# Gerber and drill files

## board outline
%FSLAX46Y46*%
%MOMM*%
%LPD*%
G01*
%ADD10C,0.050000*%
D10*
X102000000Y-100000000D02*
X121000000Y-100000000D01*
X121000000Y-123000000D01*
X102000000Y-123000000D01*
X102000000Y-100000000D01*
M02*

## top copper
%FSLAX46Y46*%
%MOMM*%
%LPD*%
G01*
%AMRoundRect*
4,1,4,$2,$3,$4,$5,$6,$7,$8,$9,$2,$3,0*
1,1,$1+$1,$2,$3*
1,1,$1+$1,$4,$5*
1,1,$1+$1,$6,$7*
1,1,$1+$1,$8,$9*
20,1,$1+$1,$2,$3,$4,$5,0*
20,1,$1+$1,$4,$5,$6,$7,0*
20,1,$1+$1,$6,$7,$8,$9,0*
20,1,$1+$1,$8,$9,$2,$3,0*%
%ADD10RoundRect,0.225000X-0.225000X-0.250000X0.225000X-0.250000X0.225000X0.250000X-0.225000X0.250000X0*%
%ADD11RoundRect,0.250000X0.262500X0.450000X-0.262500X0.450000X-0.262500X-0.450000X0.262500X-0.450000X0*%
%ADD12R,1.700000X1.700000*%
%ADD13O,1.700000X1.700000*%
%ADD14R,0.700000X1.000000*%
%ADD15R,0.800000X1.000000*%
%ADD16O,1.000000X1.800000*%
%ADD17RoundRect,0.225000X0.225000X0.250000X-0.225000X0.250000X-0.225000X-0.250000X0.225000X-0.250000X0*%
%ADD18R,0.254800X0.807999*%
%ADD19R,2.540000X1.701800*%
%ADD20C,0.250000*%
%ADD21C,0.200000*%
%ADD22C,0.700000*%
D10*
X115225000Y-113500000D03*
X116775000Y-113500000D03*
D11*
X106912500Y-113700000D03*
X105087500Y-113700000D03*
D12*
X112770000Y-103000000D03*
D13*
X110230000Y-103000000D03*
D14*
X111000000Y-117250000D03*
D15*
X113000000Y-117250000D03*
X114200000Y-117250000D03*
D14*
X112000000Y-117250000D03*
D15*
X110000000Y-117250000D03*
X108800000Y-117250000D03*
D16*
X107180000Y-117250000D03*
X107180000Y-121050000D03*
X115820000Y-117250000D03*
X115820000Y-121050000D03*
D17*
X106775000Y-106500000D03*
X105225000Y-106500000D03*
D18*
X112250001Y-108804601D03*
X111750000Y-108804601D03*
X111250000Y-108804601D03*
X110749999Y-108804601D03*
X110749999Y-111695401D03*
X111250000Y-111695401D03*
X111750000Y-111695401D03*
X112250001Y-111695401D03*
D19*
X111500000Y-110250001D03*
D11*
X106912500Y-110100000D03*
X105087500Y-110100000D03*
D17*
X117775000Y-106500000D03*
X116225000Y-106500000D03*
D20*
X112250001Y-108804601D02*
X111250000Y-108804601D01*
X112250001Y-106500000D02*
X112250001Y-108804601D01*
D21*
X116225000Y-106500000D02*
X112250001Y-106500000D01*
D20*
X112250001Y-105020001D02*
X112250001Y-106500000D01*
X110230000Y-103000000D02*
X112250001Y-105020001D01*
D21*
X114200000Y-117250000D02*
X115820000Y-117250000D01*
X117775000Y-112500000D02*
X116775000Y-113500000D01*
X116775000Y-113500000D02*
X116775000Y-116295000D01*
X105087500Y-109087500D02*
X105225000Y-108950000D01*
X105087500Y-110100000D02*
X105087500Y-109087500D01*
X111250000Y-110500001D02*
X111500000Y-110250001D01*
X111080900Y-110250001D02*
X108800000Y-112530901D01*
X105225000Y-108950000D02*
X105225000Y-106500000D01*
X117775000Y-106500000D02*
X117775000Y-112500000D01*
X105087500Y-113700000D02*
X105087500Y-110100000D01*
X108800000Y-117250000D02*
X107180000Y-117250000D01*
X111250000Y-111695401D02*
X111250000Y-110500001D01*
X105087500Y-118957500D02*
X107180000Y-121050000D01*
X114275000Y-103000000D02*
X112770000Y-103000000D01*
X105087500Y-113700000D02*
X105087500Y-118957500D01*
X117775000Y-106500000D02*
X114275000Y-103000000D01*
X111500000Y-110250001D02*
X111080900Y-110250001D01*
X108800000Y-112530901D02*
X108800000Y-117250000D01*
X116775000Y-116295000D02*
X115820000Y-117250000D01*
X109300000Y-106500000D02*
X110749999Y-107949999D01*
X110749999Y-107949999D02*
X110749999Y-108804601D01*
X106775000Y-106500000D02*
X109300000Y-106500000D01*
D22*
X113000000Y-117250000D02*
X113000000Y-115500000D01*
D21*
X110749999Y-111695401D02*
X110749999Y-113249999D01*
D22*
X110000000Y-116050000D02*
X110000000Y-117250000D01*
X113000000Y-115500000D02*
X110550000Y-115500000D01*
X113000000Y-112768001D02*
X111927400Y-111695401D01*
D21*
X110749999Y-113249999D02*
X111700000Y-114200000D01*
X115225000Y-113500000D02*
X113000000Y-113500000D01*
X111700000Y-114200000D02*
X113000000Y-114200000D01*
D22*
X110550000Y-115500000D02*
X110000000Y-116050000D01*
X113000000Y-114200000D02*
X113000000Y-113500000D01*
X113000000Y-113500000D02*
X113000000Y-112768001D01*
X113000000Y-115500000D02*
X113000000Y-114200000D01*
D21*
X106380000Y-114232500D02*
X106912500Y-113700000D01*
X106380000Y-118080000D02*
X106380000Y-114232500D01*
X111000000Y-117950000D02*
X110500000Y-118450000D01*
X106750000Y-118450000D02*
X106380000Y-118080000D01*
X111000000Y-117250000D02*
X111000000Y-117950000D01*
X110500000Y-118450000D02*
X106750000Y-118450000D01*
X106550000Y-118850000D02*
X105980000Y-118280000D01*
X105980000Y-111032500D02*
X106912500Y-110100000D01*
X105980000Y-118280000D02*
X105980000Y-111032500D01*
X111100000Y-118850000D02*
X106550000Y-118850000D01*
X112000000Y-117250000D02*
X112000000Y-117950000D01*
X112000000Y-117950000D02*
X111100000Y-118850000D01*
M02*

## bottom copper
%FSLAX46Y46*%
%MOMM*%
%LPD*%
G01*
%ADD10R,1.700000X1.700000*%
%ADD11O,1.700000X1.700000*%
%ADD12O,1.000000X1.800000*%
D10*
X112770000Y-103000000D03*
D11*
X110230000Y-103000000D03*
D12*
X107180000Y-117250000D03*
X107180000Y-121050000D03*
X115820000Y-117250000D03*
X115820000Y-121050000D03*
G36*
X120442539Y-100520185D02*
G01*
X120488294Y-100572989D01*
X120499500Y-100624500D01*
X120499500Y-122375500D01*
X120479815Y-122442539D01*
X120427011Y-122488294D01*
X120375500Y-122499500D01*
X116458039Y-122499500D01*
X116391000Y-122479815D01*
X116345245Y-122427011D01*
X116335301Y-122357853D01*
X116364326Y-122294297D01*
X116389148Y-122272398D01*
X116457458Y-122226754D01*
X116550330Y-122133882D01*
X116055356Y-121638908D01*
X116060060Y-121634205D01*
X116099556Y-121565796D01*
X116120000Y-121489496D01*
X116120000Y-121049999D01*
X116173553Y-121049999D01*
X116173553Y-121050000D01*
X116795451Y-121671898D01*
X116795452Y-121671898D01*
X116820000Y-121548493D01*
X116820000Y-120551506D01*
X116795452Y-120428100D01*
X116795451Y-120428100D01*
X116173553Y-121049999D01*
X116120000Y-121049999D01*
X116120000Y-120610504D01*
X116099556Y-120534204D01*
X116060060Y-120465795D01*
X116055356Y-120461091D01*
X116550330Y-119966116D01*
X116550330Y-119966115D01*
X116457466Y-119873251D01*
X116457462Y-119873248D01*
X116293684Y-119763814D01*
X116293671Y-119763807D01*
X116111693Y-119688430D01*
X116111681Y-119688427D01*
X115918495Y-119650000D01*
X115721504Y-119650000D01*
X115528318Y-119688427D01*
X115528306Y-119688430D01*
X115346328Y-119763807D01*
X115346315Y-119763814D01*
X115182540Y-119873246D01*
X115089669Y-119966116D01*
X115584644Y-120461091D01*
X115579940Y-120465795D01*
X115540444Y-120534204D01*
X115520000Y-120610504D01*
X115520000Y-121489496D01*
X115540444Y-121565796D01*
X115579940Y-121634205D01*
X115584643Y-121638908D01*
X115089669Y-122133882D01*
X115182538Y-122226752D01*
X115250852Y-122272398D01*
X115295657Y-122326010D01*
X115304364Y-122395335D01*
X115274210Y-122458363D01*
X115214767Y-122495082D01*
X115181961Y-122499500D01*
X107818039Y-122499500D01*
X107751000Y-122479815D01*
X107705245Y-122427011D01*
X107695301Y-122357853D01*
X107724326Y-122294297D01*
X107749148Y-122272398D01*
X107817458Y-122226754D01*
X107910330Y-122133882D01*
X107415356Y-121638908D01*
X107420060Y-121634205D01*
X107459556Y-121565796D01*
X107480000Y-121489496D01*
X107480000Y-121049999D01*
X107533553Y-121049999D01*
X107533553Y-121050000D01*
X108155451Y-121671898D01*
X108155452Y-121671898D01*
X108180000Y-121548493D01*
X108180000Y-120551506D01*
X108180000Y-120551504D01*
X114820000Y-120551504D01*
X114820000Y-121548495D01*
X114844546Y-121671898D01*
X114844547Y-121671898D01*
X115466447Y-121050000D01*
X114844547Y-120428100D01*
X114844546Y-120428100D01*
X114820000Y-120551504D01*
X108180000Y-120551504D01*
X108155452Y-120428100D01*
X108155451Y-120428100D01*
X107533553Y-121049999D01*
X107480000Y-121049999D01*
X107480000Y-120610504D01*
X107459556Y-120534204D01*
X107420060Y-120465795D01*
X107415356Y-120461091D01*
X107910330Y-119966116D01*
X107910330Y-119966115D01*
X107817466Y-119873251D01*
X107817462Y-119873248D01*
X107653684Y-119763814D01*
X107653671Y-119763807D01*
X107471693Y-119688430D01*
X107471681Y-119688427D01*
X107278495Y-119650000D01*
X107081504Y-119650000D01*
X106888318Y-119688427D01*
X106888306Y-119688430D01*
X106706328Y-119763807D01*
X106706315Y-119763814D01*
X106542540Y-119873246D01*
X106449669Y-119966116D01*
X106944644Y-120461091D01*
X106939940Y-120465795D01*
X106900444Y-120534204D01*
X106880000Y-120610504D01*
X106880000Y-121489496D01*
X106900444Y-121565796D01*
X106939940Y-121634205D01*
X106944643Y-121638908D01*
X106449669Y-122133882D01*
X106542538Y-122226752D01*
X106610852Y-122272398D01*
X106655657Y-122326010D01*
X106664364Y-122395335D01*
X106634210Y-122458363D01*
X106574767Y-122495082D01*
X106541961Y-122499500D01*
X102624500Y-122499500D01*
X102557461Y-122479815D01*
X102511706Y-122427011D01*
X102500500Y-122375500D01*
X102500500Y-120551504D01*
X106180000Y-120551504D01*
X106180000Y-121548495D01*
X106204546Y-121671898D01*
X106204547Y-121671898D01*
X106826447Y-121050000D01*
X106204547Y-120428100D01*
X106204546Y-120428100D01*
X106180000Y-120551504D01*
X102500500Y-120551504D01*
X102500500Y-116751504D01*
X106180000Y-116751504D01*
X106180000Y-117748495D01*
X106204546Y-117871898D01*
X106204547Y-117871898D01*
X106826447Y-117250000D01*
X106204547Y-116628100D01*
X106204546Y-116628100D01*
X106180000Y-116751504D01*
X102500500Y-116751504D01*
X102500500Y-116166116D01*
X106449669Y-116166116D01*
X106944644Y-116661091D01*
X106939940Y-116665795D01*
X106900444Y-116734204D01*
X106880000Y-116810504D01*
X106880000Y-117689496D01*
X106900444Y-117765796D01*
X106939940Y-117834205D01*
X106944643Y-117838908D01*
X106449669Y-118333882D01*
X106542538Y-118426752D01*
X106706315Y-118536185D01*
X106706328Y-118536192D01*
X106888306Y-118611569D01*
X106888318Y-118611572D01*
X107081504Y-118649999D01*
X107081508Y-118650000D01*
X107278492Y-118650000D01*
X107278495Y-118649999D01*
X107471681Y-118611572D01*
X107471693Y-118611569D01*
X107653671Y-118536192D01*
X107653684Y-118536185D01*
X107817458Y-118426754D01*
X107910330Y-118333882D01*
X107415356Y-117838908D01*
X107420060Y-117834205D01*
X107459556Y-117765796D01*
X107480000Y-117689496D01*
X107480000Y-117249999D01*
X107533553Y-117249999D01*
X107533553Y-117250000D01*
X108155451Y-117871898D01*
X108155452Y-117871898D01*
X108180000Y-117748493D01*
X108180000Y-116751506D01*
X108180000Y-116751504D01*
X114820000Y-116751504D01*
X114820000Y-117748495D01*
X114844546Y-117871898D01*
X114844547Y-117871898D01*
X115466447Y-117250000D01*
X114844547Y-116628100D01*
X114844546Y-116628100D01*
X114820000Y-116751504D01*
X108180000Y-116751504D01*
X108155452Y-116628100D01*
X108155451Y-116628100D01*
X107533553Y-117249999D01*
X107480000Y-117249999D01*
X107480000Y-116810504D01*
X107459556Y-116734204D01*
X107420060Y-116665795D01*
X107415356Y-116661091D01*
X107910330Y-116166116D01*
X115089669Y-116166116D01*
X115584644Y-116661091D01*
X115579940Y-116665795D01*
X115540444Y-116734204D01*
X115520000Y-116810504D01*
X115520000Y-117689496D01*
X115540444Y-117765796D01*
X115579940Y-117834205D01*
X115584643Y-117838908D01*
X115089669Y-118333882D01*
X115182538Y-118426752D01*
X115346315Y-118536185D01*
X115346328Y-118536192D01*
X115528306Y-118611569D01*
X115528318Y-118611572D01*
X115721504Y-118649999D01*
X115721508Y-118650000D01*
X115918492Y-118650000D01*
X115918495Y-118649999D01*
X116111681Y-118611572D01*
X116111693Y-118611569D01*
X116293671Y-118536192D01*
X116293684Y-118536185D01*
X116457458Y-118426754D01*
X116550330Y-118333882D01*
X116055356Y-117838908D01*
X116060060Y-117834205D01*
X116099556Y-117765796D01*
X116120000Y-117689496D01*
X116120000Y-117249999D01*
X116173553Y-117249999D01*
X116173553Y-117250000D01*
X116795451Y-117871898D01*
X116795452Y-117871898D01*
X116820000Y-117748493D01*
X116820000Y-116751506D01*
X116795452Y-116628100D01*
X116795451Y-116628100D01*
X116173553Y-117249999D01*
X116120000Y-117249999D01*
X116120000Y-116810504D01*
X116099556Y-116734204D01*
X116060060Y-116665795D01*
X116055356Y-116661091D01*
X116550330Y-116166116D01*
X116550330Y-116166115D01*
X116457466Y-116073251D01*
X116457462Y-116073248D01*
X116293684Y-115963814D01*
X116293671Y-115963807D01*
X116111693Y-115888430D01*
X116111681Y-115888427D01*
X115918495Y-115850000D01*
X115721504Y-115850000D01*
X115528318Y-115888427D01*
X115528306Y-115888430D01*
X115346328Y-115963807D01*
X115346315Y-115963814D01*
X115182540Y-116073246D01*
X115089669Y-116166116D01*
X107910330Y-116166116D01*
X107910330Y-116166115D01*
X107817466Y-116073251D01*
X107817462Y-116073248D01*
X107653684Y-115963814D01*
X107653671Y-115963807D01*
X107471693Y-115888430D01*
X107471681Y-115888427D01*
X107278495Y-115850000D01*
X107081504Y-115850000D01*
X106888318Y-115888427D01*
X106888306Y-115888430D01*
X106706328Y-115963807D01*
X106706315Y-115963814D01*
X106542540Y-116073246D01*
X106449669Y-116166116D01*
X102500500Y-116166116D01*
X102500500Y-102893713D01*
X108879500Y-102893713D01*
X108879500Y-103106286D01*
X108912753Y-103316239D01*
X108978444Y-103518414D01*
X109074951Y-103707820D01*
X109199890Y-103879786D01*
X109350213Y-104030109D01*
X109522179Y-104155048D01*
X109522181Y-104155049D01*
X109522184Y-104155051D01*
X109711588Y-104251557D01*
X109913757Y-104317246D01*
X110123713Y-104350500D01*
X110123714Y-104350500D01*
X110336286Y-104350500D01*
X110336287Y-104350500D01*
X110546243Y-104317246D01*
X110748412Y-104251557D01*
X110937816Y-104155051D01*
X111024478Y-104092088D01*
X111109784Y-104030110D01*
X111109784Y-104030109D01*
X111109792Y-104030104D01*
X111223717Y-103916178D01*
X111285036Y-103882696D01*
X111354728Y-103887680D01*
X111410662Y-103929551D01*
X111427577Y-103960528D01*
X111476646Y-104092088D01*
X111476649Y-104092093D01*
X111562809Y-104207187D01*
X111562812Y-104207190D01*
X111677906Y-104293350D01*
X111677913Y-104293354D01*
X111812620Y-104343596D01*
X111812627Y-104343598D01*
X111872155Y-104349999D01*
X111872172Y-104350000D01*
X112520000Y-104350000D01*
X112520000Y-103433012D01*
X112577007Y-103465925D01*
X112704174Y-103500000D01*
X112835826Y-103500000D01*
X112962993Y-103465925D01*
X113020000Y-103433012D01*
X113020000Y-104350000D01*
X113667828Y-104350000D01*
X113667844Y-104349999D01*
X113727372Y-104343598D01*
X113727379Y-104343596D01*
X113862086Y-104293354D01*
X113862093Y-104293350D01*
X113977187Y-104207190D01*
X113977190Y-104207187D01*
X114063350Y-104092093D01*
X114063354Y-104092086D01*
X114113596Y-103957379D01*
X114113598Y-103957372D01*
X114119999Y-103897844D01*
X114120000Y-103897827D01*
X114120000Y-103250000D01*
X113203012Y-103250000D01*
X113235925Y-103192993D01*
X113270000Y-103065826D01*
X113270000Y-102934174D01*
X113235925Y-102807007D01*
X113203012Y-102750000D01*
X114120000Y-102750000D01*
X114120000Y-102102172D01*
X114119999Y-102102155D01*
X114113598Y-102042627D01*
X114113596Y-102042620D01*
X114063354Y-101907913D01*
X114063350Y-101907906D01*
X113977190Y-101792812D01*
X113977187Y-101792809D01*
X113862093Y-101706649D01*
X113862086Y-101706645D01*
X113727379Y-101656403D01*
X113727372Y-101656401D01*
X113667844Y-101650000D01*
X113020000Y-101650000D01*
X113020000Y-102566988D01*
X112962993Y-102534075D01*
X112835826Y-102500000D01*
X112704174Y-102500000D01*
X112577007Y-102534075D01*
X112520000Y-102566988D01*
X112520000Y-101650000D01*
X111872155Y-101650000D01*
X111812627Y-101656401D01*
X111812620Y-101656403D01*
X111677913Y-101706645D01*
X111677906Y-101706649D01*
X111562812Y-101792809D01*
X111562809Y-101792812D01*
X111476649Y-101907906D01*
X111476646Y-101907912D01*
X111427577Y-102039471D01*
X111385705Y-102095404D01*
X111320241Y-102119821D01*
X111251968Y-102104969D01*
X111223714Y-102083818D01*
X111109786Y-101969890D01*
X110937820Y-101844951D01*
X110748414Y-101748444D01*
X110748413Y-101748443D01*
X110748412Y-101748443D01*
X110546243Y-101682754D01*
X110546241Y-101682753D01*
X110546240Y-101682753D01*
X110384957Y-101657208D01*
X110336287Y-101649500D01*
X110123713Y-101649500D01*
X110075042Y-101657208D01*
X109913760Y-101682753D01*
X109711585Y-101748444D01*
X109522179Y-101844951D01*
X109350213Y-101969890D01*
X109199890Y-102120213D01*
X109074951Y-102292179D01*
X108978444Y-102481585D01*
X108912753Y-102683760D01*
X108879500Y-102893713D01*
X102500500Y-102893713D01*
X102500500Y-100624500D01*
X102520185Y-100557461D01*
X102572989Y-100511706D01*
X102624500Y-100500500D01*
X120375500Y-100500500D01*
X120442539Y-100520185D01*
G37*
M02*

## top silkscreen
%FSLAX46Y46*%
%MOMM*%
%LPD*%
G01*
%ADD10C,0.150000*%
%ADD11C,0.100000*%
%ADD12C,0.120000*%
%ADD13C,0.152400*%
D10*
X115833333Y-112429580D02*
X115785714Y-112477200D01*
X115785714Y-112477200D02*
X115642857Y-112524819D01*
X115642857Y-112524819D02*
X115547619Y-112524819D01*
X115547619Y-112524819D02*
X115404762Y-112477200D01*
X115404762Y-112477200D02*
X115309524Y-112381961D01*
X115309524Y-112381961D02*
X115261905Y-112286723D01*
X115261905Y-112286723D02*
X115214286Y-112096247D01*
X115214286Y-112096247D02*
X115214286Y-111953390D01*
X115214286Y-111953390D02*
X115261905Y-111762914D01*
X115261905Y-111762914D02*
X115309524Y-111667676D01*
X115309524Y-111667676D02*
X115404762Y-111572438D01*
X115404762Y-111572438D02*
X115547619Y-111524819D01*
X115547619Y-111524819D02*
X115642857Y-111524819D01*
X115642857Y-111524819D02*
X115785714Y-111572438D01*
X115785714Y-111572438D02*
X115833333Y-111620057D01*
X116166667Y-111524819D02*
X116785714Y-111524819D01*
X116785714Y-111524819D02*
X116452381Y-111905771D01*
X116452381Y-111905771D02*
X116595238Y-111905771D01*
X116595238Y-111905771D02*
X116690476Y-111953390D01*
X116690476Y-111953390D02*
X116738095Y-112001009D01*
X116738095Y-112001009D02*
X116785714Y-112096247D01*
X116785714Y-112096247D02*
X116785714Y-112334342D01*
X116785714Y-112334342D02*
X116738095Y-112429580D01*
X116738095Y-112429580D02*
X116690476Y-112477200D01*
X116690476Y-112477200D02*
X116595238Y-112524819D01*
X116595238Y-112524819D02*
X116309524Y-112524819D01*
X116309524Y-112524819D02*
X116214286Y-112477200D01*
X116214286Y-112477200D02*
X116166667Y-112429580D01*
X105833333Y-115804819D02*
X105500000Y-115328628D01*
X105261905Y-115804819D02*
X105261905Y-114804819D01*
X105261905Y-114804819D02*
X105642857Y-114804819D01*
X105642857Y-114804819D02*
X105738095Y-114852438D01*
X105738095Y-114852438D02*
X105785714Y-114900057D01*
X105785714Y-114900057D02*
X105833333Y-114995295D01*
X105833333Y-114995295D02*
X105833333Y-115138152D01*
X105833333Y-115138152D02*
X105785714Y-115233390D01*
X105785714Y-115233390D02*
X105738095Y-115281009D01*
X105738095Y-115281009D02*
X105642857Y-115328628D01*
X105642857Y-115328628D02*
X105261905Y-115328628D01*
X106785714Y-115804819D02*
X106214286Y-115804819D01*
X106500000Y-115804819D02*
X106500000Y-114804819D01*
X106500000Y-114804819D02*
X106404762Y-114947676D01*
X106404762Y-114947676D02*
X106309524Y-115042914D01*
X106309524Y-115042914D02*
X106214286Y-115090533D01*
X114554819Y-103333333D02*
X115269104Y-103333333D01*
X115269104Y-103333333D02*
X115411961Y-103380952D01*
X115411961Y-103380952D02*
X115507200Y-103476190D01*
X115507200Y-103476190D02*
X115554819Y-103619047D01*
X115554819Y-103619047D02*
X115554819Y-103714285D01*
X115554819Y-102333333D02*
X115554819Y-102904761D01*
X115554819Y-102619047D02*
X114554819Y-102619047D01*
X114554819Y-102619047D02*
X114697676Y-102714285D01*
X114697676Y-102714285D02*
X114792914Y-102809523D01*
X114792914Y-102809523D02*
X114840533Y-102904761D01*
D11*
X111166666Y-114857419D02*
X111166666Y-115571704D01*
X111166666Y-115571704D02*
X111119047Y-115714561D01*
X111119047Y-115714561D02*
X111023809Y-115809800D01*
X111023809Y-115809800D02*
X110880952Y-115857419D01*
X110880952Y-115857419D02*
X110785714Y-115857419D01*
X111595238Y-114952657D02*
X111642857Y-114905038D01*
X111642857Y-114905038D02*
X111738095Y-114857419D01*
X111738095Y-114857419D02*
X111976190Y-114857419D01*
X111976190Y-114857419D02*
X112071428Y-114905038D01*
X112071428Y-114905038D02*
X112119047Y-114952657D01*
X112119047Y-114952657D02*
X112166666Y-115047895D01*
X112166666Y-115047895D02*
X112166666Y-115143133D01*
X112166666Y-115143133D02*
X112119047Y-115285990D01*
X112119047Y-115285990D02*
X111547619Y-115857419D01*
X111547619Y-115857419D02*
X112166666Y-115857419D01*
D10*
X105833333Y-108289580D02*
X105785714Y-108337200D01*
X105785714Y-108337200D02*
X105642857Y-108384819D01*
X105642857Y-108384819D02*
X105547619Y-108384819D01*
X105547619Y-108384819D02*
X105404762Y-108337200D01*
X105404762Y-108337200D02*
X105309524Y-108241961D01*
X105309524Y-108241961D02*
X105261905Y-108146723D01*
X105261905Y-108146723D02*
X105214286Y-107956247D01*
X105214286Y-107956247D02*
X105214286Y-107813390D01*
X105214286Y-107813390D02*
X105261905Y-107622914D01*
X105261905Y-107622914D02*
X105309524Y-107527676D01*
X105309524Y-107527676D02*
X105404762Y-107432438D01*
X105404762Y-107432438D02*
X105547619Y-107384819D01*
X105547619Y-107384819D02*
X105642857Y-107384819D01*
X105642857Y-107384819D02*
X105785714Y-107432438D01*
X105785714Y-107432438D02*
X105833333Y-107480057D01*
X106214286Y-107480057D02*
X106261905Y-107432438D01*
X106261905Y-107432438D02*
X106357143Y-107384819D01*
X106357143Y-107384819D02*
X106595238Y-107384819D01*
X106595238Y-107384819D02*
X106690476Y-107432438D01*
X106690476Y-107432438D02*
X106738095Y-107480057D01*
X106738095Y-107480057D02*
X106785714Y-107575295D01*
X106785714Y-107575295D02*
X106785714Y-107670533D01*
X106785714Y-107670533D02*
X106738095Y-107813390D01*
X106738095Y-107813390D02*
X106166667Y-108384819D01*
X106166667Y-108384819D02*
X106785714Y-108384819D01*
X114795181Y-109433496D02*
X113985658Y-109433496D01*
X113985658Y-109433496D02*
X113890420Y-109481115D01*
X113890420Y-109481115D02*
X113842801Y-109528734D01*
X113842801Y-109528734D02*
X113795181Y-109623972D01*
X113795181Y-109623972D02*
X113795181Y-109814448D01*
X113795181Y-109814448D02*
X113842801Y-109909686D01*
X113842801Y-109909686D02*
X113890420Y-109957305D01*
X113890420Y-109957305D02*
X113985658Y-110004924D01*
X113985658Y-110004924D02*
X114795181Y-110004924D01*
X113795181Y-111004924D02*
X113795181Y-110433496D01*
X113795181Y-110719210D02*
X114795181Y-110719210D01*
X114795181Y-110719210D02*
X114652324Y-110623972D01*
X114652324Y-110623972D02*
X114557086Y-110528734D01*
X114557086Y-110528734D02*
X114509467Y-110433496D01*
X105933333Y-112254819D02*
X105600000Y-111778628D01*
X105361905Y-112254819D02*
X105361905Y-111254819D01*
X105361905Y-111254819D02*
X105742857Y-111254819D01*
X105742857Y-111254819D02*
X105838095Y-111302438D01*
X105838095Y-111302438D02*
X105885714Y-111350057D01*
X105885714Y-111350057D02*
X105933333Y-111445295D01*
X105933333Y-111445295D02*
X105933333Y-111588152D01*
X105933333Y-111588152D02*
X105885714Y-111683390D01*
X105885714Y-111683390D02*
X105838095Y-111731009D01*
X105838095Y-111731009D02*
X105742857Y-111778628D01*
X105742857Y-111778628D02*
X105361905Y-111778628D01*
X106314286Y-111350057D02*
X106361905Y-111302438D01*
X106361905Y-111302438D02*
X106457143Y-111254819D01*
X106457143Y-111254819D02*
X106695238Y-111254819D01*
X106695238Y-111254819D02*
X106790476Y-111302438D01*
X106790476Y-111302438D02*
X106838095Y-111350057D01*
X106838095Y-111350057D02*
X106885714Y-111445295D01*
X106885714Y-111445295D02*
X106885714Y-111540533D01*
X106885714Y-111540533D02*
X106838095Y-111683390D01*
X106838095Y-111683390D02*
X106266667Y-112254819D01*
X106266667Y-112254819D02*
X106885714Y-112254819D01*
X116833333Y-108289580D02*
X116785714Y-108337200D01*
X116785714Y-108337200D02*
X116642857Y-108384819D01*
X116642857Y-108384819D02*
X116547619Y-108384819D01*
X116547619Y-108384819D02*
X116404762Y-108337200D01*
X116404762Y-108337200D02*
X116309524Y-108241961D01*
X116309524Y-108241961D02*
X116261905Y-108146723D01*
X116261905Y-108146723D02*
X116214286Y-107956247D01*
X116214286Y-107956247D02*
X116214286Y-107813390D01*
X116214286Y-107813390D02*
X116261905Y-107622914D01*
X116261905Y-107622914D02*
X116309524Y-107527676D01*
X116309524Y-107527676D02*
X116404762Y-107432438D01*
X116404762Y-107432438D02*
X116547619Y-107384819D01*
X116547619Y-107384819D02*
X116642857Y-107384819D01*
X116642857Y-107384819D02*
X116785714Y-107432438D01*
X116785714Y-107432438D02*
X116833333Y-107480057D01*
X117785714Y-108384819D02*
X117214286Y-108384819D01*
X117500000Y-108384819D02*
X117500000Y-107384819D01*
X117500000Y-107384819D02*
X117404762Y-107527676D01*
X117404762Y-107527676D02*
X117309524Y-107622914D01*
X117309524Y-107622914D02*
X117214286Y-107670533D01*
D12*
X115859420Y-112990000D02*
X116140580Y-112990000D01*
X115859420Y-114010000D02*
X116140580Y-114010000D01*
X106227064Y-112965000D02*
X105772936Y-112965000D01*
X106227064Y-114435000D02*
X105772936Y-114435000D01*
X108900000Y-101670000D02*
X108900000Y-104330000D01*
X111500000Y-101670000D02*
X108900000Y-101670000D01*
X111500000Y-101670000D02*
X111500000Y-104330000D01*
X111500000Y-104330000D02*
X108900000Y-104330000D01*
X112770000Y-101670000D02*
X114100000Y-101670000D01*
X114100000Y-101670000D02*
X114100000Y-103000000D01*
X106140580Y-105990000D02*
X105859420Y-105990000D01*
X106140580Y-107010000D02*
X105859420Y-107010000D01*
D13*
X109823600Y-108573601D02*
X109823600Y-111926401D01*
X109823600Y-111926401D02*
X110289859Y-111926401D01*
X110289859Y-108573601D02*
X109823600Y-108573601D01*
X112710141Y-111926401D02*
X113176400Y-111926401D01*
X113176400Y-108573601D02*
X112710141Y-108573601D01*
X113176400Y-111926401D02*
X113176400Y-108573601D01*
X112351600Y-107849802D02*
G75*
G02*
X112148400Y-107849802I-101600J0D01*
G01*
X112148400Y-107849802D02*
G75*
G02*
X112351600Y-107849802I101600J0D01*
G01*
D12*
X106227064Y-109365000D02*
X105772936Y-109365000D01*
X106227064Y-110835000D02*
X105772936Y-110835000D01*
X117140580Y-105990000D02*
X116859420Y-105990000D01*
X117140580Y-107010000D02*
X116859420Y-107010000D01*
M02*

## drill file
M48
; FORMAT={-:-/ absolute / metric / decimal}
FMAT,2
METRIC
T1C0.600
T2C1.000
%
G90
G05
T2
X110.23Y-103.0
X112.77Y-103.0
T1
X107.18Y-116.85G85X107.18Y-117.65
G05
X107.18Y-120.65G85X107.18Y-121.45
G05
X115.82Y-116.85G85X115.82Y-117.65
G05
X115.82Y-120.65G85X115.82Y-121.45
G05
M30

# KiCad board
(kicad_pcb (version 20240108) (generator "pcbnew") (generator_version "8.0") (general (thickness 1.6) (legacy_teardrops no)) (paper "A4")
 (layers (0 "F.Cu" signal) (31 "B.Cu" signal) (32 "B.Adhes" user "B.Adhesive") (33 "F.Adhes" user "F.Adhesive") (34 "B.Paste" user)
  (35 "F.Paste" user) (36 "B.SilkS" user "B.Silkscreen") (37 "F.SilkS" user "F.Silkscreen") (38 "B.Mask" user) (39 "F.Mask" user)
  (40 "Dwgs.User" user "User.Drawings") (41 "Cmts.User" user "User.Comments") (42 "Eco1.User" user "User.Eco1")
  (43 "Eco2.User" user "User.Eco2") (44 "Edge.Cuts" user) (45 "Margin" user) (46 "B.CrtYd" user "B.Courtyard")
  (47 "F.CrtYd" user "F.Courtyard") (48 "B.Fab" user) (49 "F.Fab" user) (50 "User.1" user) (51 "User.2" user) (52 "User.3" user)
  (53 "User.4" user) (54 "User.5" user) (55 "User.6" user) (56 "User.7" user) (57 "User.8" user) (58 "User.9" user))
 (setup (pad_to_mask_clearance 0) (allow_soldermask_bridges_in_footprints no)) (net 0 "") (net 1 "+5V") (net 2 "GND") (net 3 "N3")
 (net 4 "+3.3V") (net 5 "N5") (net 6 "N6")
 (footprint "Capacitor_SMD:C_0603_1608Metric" (layer "F.Cu") (at 116 113.5)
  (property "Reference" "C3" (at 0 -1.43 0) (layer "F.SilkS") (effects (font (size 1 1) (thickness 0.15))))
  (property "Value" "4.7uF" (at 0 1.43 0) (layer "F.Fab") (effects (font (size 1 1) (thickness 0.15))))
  (fp_line (start -0.14058 -0.51) (end 0.14058 -0.51) (stroke (width 0.12) (type solid)) (layer "F.SilkS"))
  (fp_line (start -0.14058 0.51) (end 0.14058 0.51) (stroke (width 0.12) (type solid)) (layer "F.SilkS"))
  (pad "1" smd roundrect (at -0.775 0) (size 0.9 0.95) (layers "F.Cu" "F.Paste" "F.Mask") (roundrect_rratio 0.25) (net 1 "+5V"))
  (pad "2" smd roundrect (at 0.775 0) (size 0.9 0.95) (layers "F.Cu" "F.Paste" "F.Mask") (roundrect_rratio 0.25) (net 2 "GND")))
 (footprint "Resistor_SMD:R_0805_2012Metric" (layer "F.Cu") (at 106 113.7 180)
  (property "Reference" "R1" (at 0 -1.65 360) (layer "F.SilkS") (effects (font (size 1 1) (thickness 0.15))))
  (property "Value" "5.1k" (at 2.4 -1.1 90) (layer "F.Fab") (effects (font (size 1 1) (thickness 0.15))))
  (fp_line (start -0.227064 0.735) (end 0.227064 0.735) (stroke (width 0.12) (type solid)) (layer "F.SilkS"))
  (fp_line (start -0.227064 -0.735) (end 0.227064 -0.735) (stroke (width 0.12) (type solid)) (layer "F.SilkS"))
  (pad "1" smd roundrect (at -0.9125 0 180) (size 1.025 1.4) (layers "F.Cu" "F.Paste" "F.Mask") (roundrect_rratio 0.243902) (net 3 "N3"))
  (pad "2" smd roundrect (at 0.9125 0 180) (size 1.025 1.4) (layers "F.Cu" "F.Paste" "F.Mask") (roundrect_rratio 0.243902) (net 2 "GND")))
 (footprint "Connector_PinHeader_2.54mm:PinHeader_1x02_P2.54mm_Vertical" (layer "F.Cu") (at 112.77 103 -90)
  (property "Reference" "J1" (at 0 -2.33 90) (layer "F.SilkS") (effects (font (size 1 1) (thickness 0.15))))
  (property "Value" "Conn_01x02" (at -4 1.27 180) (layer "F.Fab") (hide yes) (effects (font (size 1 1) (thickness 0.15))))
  (fp_line (start -1.33 3.87) (end 1.33 3.87) (stroke (width 0.12) (type solid)) (layer "F.SilkS"))
  (fp_line (start -1.33 1.27) (end -1.33 3.87) (stroke (width 0.12) (type solid)) (layer "F.SilkS"))
  (fp_line (start -1.33 1.27) (end 1.33 1.27) (stroke (width 0.12) (type solid)) (layer "F.SilkS"))
  (fp_line (start 1.33 1.27) (end 1.33 3.87) (stroke (width 0.12) (type solid)) (layer "F.SilkS"))
  (fp_line (start -1.33 0) (end -1.33 -1.33) (stroke (width 0.12) (type solid)) (layer "F.SilkS"))
  (fp_line (start -1.33 -1.33) (end 0 -1.33) (stroke (width 0.12) (type solid)) (layer "F.SilkS"))
  (pad "1" thru_hole rect (at 0 0 270) (size 1.7 1.7) (drill 1) (layers "*.Cu" "*.Mask") (remove_unused_layers no) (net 2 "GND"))
  (pad "2" thru_hole oval (at 0 2.54 270) (size 1.7 1.7) (drill 1) (layers "*.Cu" "*.Mask") (remove_unused_layers no) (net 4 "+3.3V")))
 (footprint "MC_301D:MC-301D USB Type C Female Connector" (layer "F.Cu") (at 111.5 120)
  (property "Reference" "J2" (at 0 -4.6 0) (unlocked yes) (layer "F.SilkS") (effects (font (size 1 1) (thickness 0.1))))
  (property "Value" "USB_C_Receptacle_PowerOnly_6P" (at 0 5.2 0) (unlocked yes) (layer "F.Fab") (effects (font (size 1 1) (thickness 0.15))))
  (pad "A5" smd rect (at -0.5 -2.75) (size 0.7 1) (layers "F.Cu" "F.Paste" "F.Mask") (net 3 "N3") (thermal_bridge_angle 45))
  (pad "A9" smd rect (at 1.5 -2.75) (size 0.8 1) (layers "F.Cu" "F.Paste" "F.Mask") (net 1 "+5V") (thermal_bridge_angle 45))
  (pad "A12" smd rect (at 2.7 -2.75) (size 0.8 1) (layers "F.Cu" "F.Paste" "F.Mask") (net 2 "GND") (thermal_bridge_angle 45))
  (pad "B5" smd rect (at 0.5 -2.75) (size 0.7 1) (layers "F.Cu" "F.Paste" "F.Mask") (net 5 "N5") (thermal_bridge_angle 45))
  (pad "B9" smd rect (at -1.5 -2.75) (size 0.8 1) (layers "F.Cu" "F.Paste" "F.Mask") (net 1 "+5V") (thermal_bridge_angle 45))
  (pad "B12" smd rect (at -2.7 -2.75) (size 0.8 1) (layers "F.Cu" "F.Paste" "F.Mask") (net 2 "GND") (thermal_bridge_angle 45))
  (pad "S1" thru_hole oval (at -4.32 -2.75) (size 1 1.8) (drill oval 0.6 1.4) (layers "*.Cu" "*.Mask") (remove_unused_layers no)
   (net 2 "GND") (thermal_bridge_angle 45))
  (pad "S1" thru_hole oval (at -4.32 1.05) (size 1 1.8) (drill oval 0.6 1.4) (layers "*.Cu" "*.Mask") (remove_unused_layers no)
   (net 2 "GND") (thermal_bridge_angle 45))
  (pad "S1" thru_hole oval (at 4.32 -2.75) (size 1 1.8) (drill oval 0.6 1.4) (layers "*.Cu" "*.Mask") (remove_unused_layers no)
   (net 2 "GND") (thermal_bridge_angle 45))
  (pad "S1" thru_hole oval (at 4.32 1.05) (size 1 1.8) (drill oval 0.6 1.4) (layers "*.Cu" "*.Mask") (remove_unused_layers no) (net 2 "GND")
   (thermal_bridge_angle 45)))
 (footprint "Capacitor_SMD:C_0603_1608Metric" (layer "F.Cu") (at 106 106.5 180)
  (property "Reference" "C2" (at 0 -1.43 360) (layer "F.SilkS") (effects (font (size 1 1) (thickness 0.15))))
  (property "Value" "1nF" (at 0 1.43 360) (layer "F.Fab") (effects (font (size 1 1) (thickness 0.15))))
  (fp_line (start -0.14058 0.51) (end 0.14058 0.51) (stroke (width 0.12) (type solid)) (layer "F.SilkS"))
  (fp_line (start -0.14058 -0.51) (end 0.14058 -0.51) (stroke (width 0.12) (type solid)) (layer "F.SilkS"))
  (pad "1" smd roundrect (at -0.775 0 180) (size 0.9 0.95) (layers "F.Cu" "F.Paste" "F.Mask") (roundrect_rratio 0.25) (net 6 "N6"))
  (pad "2" smd roundrect (at 0.775 0 180) (size 0.9 0.95) (layers "F.Cu" "F.Paste" "F.Mask") (roundrect_rratio 0.25) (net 2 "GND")))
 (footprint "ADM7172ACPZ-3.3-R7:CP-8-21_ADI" (layer "F.Cu") (at 111.5 110.250001 -90)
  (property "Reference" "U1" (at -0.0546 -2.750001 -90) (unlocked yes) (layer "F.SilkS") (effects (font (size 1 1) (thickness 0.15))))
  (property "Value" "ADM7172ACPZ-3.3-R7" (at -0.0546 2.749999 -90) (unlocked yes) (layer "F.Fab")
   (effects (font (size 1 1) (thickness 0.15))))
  (fp_line (start -1.6764 1.6764) (end 1.6764 1.6764) (stroke (width 0.1524) (type solid)) (layer "F.SilkS"))
  (fp_line (start 1.6764 1.6764) (end 1.6764 1.210141) (stroke (width 0.1524) (type solid)) (layer "F.SilkS"))
  (fp_line (start -1.6764 1.210141) (end -1.6764 1.6764) (stroke (width 0.1524) (type solid)) (layer "F.SilkS"))
  (fp_line (start 1.6764 -1.210141) (end 1.6764 -1.6764) (stroke (width 0.1524) (type solid)) (layer "F.SilkS"))
  (fp_line (start -1.6764 -1.6764) (end -1.6764 -1.210141) (stroke (width 0.1524) (type solid)) (layer "F.SilkS"))
  (fp_line (start 1.6764 -1.6764) (end -1.6764 -1.6764) (stroke (width 0.1524) (type solid)) (layer "F.SilkS"))
  (fp_circle (center -2.400199 -0.75) (end -2.298599 -0.75) (stroke (width 0.1524) (type solid)) (fill none) (layer "F.SilkS"))
  (pad "1" smd rect (at -1.4454 -0.750001 270) (size 0.807999 0.2548) (layers "F.Cu" "F.Paste" "F.Mask") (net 4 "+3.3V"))
  (pad "2" smd rect (at -1.4454 -0.25 270) (size 0.807999 0.2548) (layers "F.Cu" "F.Paste" "F.Mask") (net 4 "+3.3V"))
  (pad "3" smd rect (at -1.4454 0.25 270) (size 0.807999 0.2548) (layers "F.Cu" "F.Paste" "F.Mask") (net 4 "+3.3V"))
  (pad "4" smd rect (at -1.4454 0.750001 270) (size 0.807999 0.2548) (layers "F.Cu" "F.Paste" "F.Mask") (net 6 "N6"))
  (pad "5" smd rect (at 1.4454 0.750001 270) (size 0.807999 0.2548) (layers "F.Cu" "F.Paste" "F.Mask") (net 1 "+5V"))
  (pad "6" smd rect (at 1.4454 0.25 270) (size 0.807999 0.2548) (layers "F.Cu" "F.Paste" "F.Mask") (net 2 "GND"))
  (pad "7" smd rect (at 1.4454 -0.25 270) (size 0.807999 0.2548) (layers "F.Cu" "F.Paste" "F.Mask") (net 1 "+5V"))
  (pad "8" smd rect (at 1.4454 -0.750001 270) (size 0.807999 0.2548) (layers "F.Cu" "F.Paste" "F.Mask") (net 1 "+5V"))
  (pad "9" smd rect (at 0 0 270) (size 1.7018 2.54) (layers "F.Cu" "F.Paste" "F.Mask") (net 2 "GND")))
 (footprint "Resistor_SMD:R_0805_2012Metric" (layer "F.Cu") (at 106 110.1 180)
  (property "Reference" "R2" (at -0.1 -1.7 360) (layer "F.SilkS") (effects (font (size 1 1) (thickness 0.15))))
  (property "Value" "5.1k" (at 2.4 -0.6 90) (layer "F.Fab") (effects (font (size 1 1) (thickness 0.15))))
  (fp_line (start -0.227064 0.735) (end 0.227064 0.735) (stroke (width 0.12) (type solid)) (layer "F.SilkS"))
  (fp_line (start -0.227064 -0.735) (end 0.227064 -0.735) (stroke (width 0.12) (type solid)) (layer "F.SilkS"))
  (pad "1" smd roundrect (at -0.9125 0 180) (size 1.025 1.4) (layers "F.Cu" "F.Paste" "F.Mask") (roundrect_rratio 0.243902) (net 5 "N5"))
  (pad "2" smd roundrect (at 0.9125 0 180) (size 1.025 1.4) (layers "F.Cu" "F.Paste" "F.Mask") (roundrect_rratio 0.243902) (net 2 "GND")))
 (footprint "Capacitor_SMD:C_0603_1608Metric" (layer "F.Cu") (at 117 106.5 180)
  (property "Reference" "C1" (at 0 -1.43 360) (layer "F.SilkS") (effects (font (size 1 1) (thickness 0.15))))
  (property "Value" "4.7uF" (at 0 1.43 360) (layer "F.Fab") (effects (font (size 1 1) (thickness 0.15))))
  (fp_line (start -0.14058 0.51) (end 0.14058 0.51) (stroke (width 0.12) (type solid)) (layer "F.SilkS"))
  (fp_line (start -0.14058 -0.51) (end 0.14058 -0.51) (stroke (width 0.12) (type solid)) (layer "F.SilkS"))
  (pad "1" smd roundrect (at -0.775 0 180) (size 0.9 0.95) (layers "F.Cu" "F.Paste" "F.Mask") (roundrect_rratio 0.25) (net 2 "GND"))
  (pad "2" smd roundrect (at 0.775 0 180) (size 0.9 0.95) (layers "F.Cu" "F.Paste" "F.Mask") (roundrect_rratio 0.25) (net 4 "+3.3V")))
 (gr_rect (start 102 100) (end 121 123) (stroke (width 0.05) (type default)) (fill none) (layer "Edge.Cuts"))
 (segment (start 112.250001 108.804601) (end 111.25 108.804601) (width 0.25) (layer "F.Cu") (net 4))
 (segment (start 112.250001 106.5) (end 112.250001 108.804601) (width 0.25) (layer "F.Cu") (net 4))
 (segment (start 116.225 106.5) (end 112.250001 106.5) (width 0.2) (layer "F.Cu") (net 4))
 (segment (start 112.250001 105.020001) (end 112.250001 106.5) (width 0.25) (layer "F.Cu") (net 4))
 (segment (start 110.23 103) (end 112.250001 105.020001) (width 0.25) (layer "F.Cu") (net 4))
 (segment (start 114.2 117.25) (end 115.82 117.25) (width 0.2) (layer "F.Cu") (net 2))
 (segment (start 117.775 112.5) (end 116.775 113.5) (width 0.2) (layer "F.Cu") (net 2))
 (segment (start 116.775 113.5) (end 116.775 116.295) (width 0.2) (layer "F.Cu") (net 2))
 (segment (start 105.0875 109.0875) (end 105.225 108.95) (width 0.2) (layer "F.Cu") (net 2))
 (segment (start 105.0875 110.1) (end 105.0875 109.0875) (width 0.2) (layer "F.Cu") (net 2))
 (segment (start 111.25 110.500001) (end 111.5 110.250001) (width 0.2) (layer "F.Cu") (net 2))
 (segment (start 111.0809 110.250001) (end 108.8 112.530901) (width 0.2) (layer "F.Cu") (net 2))
 (segment (start 105.225 108.95) (end 105.225 106.5) (width 0.2) (layer "F.Cu") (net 2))
 (segment (start 117.775 106.5) (end 117.775 112.5) (width 0.2) (layer "F.Cu") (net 2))
 (segment (start 105.0875 113.7) (end 105.0875 110.1) (width 0.2) (layer "F.Cu") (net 2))
 (segment (start 108.8 117.25) (end 107.18 117.25) (width 0.2) (layer "F.Cu") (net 2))
 (segment (start 111.25 111.695401) (end 111.25 110.500001) (width 0.2) (layer "F.Cu") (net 2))
 (segment (start 105.0875 118.9575) (end 107.18 121.05) (width 0.2) (layer "F.Cu") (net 2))
 (segment (start 114.275 103) (end 112.77 103) (width 0.2) (layer "F.Cu") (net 2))
 (segment (start 105.0875 113.7) (end 105.0875 118.9575) (width 0.2) (layer "F.Cu") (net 2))
 (segment (start 117.775 106.5) (end 114.275 103) (width 0.2) (layer "F.Cu") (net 2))
 (segment (start 111.5 110.250001) (end 111.0809 110.250001) (width 0.2) (layer "F.Cu") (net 2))
 (segment (start 108.8 112.530901) (end 108.8 117.25) (width 0.2) (layer "F.Cu") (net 2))
 (segment (start 116.775 116.295) (end 115.82 117.25) (width 0.2) (layer "F.Cu") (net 2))
 (segment (start 109.3 106.5) (end 110.749999 107.949999) (width 0.2) (layer "F.Cu") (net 6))
 (segment (start 110.749999 107.949999) (end 110.749999 108.804601) (width 0.2) (layer "F.Cu") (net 6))
 (segment (start 106.775 106.5) (end 109.3 106.5) (width 0.2) (layer "F.Cu") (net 6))
 (segment (start 113 117.25) (end 113 115.5) (width 0.7) (layer "F.Cu") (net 1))
 (segment (start 110.749999 111.695401) (end 110.749999 113.249999) (width 0.2) (layer "F.Cu") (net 1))
 (segment (start 110 116.05) (end 110 117.25) (width 0.7) (layer "F.Cu") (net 1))
 (segment (start 113 115.5) (end 110.55 115.5) (width 0.7) (layer "F.Cu") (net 1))
 (segment (start 113 112.768001) (end 111.9274 111.695401) (width 0.7) (layer "F.Cu") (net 1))
 (segment (start 110.749999 113.249999) (end 111.7 114.2) (width 0.2) (layer "F.Cu") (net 1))
 (segment (start 115.225 113.5) (end 113 113.5) (width 0.2) (layer "F.Cu") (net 1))
 (segment (start 111.7 114.2) (end 113 114.2) (width 0.2) (layer "F.Cu") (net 1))
 (segment (start 110.55 115.5) (end 110 116.05) (width 0.7) (layer "F.Cu") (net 1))
 (segment (start 113 114.2) (end 113 113.5) (width 0.7) (layer "F.Cu") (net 1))
 (segment (start 113 113.5) (end 113 112.768001) (width 0.7) (layer "F.Cu") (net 1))
 (segment (start 113 115.5) (end 113 114.2) (width 0.7) (layer "F.Cu") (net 1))
 (segment (start 106.38 114.2325) (end 106.9125 113.7) (width 0.2) (layer "F.Cu") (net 3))
 (segment (start 106.38 118.08) (end 106.38 114.2325) (width 0.2) (layer "F.Cu") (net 3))
 (segment (start 111 117.95) (end 110.5 118.45) (width 0.2) (layer "F.Cu") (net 3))
 (segment (start 106.75 118.45) (end 106.38 118.08) (width 0.2) (layer "F.Cu") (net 3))
 (segment (start 111 117.25) (end 111 117.95) (width 0.2) (layer "F.Cu") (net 3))
 (segment (start 110.5 118.45) (end 106.75 118.45) (width 0.2) (layer "F.Cu") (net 3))
 (segment (start 106.55 118.85) (end 105.98 118.28) (width 0.2) (layer "F.Cu") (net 5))
 (segment (start 105.98 111.0325) (end 106.9125 110.1) (width 0.2) (layer "F.Cu") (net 5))
 (segment (start 105.98 118.28) (end 105.98 111.0325) (width 0.2) (layer "F.Cu") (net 5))
 (segment (start 111.1 118.85) (end 106.55 118.85) (width 0.2) (layer "F.Cu") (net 5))
 (segment (start 112 117.25) (end 112 117.95) (width 0.2) (layer "F.Cu") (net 5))
 (segment (start 112 117.95) (end 111.1 118.85) (width 0.2) (layer "F.Cu") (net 5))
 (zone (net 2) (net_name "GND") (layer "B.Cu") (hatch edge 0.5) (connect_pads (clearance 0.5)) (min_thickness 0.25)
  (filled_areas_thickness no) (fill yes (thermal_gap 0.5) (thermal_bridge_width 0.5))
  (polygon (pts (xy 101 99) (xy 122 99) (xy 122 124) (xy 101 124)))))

